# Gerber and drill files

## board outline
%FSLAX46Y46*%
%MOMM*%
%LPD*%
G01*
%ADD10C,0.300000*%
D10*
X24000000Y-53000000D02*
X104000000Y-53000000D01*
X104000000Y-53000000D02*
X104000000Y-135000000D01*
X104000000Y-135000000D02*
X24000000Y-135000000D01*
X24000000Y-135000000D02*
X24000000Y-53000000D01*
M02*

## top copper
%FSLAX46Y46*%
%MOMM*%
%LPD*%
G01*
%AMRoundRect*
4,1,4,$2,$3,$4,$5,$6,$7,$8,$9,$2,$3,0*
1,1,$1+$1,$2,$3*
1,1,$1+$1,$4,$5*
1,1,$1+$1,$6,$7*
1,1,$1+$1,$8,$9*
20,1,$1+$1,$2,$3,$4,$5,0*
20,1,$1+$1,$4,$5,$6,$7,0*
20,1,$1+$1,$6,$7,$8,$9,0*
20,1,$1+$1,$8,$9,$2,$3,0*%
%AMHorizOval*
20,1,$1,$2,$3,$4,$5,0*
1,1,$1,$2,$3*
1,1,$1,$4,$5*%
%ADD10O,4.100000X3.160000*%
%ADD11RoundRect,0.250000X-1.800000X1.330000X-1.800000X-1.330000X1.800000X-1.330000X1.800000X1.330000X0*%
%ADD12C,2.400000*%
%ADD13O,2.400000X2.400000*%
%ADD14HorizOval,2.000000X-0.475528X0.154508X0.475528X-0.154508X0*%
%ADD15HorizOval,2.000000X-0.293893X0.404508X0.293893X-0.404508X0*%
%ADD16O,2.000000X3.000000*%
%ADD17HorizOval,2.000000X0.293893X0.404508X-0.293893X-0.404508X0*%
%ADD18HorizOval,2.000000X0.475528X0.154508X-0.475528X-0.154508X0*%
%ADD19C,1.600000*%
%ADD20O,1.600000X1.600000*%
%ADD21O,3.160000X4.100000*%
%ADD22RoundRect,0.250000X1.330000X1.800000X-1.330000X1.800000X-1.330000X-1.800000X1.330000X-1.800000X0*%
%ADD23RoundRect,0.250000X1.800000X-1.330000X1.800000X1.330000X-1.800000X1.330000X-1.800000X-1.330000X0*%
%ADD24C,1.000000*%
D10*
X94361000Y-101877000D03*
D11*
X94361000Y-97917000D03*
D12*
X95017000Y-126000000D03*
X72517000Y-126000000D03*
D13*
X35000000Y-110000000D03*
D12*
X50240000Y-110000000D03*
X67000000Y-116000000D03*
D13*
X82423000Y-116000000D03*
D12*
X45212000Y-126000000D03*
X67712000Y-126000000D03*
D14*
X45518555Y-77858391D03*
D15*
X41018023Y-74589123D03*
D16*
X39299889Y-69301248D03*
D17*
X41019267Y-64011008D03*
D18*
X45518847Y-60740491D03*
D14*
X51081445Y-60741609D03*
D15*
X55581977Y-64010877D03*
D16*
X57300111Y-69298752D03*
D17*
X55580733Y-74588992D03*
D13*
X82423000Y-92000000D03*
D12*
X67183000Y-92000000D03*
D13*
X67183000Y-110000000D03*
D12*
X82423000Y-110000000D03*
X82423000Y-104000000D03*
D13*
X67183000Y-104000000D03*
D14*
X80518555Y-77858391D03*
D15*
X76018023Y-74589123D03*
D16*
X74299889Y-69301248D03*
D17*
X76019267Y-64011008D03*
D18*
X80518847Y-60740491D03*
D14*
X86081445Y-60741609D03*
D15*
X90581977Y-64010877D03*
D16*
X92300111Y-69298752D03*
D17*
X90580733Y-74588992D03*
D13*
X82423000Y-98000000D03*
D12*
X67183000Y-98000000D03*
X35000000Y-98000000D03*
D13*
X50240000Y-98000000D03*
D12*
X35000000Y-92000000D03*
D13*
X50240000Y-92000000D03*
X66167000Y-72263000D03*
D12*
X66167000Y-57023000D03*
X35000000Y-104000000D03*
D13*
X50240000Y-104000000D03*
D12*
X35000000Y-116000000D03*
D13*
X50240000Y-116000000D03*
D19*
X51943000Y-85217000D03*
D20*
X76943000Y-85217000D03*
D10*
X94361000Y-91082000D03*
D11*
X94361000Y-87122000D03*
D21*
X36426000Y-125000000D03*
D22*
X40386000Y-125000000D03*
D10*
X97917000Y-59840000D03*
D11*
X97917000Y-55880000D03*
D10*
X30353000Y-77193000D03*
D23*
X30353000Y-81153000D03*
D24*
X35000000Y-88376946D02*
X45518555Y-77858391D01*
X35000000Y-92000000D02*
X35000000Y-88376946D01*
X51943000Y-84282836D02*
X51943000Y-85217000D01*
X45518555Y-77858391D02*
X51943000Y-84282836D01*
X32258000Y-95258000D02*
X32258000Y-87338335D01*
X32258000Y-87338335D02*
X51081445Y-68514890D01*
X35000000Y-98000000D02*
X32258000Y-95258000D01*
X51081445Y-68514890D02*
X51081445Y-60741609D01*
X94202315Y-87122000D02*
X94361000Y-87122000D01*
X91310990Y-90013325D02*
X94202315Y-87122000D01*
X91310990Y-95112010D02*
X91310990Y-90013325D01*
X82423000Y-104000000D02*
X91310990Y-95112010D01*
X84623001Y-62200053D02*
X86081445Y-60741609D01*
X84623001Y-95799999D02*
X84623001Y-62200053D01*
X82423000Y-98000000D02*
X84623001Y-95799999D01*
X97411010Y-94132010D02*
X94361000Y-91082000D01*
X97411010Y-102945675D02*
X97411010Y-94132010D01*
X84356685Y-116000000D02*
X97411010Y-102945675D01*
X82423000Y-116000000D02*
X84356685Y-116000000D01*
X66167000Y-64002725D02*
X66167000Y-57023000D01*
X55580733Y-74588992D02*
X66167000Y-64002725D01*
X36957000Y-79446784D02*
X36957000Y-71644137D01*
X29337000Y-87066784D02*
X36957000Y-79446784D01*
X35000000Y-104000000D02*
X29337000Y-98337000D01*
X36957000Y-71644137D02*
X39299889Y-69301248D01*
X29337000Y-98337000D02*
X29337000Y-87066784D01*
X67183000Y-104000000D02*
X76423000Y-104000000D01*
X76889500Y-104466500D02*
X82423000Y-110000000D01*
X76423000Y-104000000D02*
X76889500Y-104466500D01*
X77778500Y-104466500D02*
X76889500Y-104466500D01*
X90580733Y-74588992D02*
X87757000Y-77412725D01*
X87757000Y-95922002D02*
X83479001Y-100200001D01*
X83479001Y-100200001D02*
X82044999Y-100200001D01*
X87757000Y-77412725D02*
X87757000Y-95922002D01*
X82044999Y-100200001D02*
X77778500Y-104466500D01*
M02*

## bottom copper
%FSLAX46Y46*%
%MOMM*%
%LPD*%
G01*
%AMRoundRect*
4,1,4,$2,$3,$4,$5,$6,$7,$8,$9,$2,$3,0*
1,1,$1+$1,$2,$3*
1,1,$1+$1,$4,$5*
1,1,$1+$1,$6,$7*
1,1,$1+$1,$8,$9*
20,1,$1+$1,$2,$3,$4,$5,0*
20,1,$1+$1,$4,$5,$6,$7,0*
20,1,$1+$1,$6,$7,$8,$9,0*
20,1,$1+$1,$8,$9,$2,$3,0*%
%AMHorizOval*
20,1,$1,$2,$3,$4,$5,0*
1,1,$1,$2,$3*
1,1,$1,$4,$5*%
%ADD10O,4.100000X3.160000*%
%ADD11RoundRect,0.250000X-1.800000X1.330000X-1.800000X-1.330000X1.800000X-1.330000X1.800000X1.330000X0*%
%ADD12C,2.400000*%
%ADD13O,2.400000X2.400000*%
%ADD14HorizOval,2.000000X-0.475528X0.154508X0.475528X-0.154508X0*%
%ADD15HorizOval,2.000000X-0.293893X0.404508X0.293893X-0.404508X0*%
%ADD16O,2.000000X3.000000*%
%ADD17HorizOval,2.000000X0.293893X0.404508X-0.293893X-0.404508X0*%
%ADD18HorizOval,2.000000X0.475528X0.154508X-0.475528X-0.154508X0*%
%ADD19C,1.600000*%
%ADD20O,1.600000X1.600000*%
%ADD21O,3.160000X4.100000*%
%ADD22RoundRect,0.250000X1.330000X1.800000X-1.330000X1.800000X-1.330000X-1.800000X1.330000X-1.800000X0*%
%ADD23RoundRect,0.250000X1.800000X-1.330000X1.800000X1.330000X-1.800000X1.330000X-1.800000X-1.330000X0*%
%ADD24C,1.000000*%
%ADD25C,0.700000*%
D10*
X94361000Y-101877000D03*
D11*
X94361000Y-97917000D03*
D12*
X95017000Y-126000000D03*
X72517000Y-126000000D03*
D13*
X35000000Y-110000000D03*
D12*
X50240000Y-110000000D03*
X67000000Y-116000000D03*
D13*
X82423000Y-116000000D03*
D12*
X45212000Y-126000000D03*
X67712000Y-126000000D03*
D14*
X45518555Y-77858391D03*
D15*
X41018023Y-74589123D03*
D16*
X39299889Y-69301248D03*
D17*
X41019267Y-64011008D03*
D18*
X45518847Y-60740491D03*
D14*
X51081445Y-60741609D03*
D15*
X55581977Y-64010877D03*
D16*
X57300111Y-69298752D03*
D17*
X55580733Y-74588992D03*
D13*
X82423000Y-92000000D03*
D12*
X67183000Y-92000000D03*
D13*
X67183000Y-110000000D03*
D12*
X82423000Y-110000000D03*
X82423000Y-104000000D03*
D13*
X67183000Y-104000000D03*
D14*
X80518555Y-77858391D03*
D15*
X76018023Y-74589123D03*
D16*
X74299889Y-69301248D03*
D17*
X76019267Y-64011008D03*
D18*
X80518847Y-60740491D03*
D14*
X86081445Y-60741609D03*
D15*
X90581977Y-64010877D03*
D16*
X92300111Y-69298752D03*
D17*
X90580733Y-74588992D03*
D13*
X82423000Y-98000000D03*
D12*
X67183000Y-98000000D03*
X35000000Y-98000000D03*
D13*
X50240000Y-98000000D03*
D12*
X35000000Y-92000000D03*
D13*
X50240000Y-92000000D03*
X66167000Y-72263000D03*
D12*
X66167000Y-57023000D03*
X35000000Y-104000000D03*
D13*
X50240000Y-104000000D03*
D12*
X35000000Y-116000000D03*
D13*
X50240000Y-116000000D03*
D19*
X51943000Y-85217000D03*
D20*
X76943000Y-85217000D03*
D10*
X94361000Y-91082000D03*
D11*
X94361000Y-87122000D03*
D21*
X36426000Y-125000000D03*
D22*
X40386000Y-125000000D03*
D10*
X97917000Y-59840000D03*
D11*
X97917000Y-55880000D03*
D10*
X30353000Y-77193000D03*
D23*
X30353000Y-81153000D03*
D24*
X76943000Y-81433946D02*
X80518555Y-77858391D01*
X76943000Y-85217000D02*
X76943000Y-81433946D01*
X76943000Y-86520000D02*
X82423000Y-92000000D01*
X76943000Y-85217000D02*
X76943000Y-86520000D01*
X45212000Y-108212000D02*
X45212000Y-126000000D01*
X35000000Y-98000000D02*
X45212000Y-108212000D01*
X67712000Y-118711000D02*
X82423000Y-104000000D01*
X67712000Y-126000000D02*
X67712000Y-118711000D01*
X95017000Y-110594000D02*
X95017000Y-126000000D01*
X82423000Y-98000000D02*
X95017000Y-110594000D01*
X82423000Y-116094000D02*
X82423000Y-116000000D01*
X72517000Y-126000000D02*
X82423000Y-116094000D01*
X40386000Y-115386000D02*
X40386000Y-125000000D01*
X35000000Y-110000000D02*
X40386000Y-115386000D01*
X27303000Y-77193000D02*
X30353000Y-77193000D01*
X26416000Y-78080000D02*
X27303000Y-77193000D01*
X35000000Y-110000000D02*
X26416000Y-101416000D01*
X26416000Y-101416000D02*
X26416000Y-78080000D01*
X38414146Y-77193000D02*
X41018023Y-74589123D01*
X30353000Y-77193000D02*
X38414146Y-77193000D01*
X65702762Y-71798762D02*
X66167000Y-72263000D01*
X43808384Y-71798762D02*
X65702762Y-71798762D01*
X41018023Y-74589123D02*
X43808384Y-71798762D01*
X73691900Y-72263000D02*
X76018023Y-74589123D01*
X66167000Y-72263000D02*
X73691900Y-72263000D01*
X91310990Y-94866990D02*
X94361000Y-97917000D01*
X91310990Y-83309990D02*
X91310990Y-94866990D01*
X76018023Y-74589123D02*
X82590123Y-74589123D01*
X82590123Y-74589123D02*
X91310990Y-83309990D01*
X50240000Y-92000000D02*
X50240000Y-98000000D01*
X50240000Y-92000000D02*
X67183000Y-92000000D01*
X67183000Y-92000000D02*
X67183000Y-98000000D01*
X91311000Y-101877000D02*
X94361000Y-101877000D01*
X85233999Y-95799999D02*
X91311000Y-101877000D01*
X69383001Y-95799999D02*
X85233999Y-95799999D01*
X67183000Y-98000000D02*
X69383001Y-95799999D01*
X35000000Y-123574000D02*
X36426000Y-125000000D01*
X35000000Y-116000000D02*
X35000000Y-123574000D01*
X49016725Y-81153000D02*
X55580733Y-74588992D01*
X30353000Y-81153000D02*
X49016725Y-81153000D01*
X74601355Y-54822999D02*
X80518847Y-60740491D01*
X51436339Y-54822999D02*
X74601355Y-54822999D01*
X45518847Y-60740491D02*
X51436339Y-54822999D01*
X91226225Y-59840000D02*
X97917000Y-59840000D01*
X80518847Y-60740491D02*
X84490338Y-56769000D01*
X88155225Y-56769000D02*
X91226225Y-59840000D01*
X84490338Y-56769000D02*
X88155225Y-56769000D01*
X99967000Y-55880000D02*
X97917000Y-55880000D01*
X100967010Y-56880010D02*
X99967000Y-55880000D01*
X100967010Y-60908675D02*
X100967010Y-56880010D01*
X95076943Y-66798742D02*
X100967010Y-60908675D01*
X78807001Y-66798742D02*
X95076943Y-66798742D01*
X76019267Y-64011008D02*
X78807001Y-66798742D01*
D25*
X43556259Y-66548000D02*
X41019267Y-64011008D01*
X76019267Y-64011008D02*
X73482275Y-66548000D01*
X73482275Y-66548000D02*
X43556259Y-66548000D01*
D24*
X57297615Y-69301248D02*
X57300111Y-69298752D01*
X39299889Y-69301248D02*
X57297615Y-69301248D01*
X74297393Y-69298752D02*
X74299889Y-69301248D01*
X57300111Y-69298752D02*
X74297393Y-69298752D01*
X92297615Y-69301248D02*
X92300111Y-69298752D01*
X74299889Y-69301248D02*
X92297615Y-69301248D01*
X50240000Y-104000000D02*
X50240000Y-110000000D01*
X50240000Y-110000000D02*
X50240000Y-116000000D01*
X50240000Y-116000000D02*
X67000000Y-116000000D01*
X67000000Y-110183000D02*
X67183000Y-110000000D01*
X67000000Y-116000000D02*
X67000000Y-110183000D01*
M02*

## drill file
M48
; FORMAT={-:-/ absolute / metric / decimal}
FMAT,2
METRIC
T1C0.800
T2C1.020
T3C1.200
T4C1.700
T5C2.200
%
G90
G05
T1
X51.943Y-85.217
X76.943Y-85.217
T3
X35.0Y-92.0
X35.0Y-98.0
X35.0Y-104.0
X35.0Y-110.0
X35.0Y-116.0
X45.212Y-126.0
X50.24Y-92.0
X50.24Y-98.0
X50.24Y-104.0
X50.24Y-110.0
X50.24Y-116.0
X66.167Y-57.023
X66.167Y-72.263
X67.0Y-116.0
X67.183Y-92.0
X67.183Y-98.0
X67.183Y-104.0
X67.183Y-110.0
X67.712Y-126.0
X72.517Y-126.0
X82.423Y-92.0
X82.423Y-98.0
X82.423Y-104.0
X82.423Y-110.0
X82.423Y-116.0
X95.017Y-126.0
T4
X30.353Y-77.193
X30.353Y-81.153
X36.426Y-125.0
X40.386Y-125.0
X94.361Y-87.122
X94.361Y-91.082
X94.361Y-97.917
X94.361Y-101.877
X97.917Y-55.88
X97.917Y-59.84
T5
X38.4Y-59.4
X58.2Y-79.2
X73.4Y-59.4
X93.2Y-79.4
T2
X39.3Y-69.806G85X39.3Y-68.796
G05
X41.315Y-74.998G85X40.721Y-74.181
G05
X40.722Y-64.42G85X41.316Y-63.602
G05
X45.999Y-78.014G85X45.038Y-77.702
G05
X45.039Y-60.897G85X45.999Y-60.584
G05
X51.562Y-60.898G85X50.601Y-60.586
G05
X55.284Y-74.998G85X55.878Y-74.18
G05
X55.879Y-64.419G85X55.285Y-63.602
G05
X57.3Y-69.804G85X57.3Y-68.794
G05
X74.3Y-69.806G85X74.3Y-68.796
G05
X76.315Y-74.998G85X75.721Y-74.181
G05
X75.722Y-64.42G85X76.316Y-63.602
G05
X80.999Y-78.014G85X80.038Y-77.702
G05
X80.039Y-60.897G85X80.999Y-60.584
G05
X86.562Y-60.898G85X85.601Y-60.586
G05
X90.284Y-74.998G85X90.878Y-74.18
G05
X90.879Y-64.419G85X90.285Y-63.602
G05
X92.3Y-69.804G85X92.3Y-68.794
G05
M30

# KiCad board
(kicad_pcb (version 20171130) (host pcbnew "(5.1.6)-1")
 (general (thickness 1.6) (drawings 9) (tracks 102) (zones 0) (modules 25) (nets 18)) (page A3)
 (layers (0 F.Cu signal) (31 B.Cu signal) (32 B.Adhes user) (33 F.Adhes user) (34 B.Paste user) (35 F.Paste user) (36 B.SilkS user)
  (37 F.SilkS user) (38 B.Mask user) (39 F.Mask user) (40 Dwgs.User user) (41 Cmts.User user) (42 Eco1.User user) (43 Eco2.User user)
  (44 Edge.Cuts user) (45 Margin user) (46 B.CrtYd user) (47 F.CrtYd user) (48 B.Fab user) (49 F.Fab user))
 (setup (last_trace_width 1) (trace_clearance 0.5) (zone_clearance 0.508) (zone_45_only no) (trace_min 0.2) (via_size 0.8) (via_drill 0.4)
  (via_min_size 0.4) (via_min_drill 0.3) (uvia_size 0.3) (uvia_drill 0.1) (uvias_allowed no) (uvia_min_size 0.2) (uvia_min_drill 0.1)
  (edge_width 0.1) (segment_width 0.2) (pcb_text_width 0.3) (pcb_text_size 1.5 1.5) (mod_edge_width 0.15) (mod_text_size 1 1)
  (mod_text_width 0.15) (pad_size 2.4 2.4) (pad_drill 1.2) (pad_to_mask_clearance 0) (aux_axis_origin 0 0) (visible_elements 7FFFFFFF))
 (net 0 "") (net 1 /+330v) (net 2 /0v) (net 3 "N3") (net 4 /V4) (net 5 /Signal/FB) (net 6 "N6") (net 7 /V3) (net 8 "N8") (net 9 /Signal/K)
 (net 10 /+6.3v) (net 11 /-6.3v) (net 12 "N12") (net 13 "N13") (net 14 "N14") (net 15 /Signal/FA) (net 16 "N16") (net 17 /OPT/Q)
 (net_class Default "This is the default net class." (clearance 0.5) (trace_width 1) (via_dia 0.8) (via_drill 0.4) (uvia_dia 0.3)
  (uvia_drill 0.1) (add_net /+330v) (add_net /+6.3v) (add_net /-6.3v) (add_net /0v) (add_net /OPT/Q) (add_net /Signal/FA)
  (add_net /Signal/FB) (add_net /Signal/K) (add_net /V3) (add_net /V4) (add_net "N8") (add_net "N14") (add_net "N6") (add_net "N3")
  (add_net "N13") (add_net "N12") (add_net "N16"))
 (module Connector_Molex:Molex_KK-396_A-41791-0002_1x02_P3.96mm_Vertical (layer F.Cu) (at 94.361 97.917 270)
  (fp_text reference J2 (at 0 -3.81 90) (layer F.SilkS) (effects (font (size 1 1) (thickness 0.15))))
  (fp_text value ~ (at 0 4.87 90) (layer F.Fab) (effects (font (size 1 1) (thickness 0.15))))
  (pad 2 thru_hole oval (at 3.96 0 270) (size 3.16 4.1) (drill 1.7) (layers *.Cu *.Mask) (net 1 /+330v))
  (pad 1 thru_hole roundrect (at 0 0 270) (size 3.16 4.1) (drill 1.7) (layers *.Cu *.Mask) (roundrect_rratio 0.079114) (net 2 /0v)))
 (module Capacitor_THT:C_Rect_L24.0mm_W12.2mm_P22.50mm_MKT (layer F.Cu) (at 72.517 126)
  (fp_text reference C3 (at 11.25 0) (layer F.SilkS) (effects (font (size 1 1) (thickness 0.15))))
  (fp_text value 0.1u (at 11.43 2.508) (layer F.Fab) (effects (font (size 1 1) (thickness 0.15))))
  (pad 2 thru_hole circle (at 22.5 0) (size 2.4 2.4) (drill 1.2) (layers *.Cu *.Mask) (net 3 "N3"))
  (pad 1 thru_hole circle (at 0 0) (size 2.4 2.4) (drill 1.2) (layers *.Cu *.Mask) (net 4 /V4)))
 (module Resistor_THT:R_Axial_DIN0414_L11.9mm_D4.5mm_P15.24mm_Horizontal (layer F.Cu) (at 50.24 110 180)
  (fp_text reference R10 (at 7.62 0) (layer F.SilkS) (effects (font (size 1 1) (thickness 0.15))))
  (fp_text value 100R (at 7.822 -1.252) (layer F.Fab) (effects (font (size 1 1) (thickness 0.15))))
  (pad 2 thru_hole oval (at 15.24 0 180) (size 2.4 2.4) (drill 1.2) (layers *.Cu *.Mask) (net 2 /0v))
  (pad 1 thru_hole circle (at 0 0 180) (size 2.4 2.4) (drill 1.2) (layers *.Cu *.Mask) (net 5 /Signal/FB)))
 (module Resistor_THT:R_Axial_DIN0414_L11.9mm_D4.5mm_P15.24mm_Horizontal (layer F.Cu) (at 67.183 116)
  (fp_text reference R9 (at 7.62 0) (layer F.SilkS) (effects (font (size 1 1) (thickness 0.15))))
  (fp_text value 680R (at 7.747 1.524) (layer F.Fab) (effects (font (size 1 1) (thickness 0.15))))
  (pad 1 thru_hole circle (at -0.183 0) (size 2.4 2.4) (drill 1.2) (layers *.Cu *.Mask) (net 5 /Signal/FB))
  (pad 2 thru_hole oval (at 15.24 0) (size 2.4 2.4) (drill 1.2) (layers *.Cu *.Mask) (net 4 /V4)))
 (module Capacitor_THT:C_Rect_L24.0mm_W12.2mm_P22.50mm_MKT (layer F.Cu) (at 45.212 126)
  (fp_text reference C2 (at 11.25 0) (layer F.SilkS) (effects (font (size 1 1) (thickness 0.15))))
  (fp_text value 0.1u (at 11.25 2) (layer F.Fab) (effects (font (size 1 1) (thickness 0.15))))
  (pad 1 thru_hole circle (at 0 0) (size 2.4 2.4) (drill 1.2) (layers *.Cu *.Mask) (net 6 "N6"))
  (pad 2 thru_hole circle (at 22.5 0) (size 2.4 2.4) (drill 1.2) (layers *.Cu *.Mask) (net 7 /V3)))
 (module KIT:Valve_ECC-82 (layer B.Cu) (at 48.3 69.3 198)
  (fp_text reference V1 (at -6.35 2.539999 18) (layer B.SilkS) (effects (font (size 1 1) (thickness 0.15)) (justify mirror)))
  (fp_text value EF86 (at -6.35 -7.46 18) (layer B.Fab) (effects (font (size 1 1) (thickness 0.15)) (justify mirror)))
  (pad 1 thru_hole oval (at 5.29 -7.28 252) (size 2 3) (drill oval 1.02 2.03) (layers *.Cu *.Mask) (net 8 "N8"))
  (pad 2 thru_hole oval (at 8.56 -2.78 216) (size 2 3) (drill oval 1.02 2.03) (layers *.Cu *.Mask) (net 2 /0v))
  (pad 3 thru_hole oval (at 8.56 2.78 180) (size 2 3) (drill oval 1.02 2.03) (layers *.Cu *.Mask) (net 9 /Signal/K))
  (pad 4 thru_hole oval (at 5.29 7.28 144) (size 2 3) (drill oval 1.02 2.03) (layers *.Cu *.Mask) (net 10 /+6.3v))
  (pad 5 thru_hole oval (at 0 9 108) (size 2 3) (drill oval 1.02 2.03) (layers *.Cu *.Mask) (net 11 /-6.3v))
  (pad 6 thru_hole oval (at -5.29 7.28 252) (size 2 3) (drill oval 1.02 2.03) (layers *.Cu *.Mask) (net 6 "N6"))
  (pad 7 thru_hole oval (at -8.56 2.78 216) (size 2 3) (drill oval 1.02 2.03) (layers *.Cu *.Mask) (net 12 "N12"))
  (pad 8 thru_hole oval (at -8.56 -2.78 180) (size 2 3) (drill oval 1.02 2.03) (layers *.Cu *.Mask) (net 9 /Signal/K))
  (pad 9 thru_hole oval (at -5.29 -7.28 144) (size 2 3) (drill oval 1.02 2.03) (layers *.Cu *.Mask) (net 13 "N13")))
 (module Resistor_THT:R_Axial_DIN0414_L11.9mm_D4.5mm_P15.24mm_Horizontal (layer F.Cu) (at 67.183 92)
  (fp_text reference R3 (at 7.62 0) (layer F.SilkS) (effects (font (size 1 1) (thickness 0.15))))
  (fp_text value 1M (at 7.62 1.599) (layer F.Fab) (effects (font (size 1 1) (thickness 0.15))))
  (pad 2 thru_hole oval (at 15.24 0) (size 2.4 2.4) (drill 1.2) (layers *.Cu *.Mask) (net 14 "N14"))
  (pad 1 thru_hole circle (at 0 0) (size 2.4 2.4) (drill 1.2) (layers *.Cu *.Mask) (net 1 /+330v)))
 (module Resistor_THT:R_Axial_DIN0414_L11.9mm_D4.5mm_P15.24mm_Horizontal (layer F.Cu) (at 82.423 110 180)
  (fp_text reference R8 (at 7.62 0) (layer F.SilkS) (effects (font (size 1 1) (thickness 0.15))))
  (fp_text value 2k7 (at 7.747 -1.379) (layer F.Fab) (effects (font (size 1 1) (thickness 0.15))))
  (pad 2 thru_hole oval (at 15.24 0 180) (size 2.4 2.4) (drill 1.2) (layers *.Cu *.Mask) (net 5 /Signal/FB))
  (pad 1 thru_hole circle (at 0 0 180) (size 2.4 2.4) (drill 1.2) (layers *.Cu *.Mask) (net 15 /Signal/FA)))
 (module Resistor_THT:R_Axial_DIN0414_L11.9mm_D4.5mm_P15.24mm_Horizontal (layer F.Cu) (at 82.423 104 180)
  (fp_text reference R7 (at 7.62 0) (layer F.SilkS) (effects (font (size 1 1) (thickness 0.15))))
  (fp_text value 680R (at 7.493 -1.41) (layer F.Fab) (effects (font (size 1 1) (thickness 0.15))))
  (pad 1 thru_hole circle (at 0 0 180) (size 2.4 2.4) (drill 1.2) (layers *.Cu *.Mask) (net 7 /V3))
  (pad 2 thru_hole oval (at 15.24 0 180) (size 2.4 2.4) (drill 1.2) (layers *.Cu *.Mask) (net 15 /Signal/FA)))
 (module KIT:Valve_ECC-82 (layer B.Cu) (at 83.3 69.3 198)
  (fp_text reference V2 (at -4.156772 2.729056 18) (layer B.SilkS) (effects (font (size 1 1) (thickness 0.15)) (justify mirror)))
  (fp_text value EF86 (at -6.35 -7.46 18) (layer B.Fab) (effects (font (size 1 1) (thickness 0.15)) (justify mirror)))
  (pad 1 thru_hole oval (at 5.29 -7.28 252) (size 2 3) (drill oval 1.02 2.03) (layers *.Cu *.Mask) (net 14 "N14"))
  (pad 2 thru_hole oval (at 8.56 -2.78 216) (size 2 3) (drill oval 1.02 2.03) (layers *.Cu *.Mask) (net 2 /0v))
  (pad 3 thru_hole oval (at 8.56 2.78 180) (size 2 3) (drill oval 1.02 2.03) (layers *.Cu *.Mask) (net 9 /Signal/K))
  (pad 4 thru_hole oval (at 5.29 7.28 144) (size 2 3) (drill oval 1.02 2.03) (layers *.Cu *.Mask) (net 10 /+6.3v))
  (pad 5 thru_hole oval (at 0 9 108) (size 2 3) (drill oval 1.02 2.03) (layers *.Cu *.Mask) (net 11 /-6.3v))
  (pad 6 thru_hole oval (at -5.29 7.28 252) (size 2 3) (drill oval 1.02 2.03) (layers *.Cu *.Mask) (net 3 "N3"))
  (pad 7 thru_hole oval (at -8.56 2.78 216) (size 2 3) (drill oval 1.02 2.03) (layers *.Cu *.Mask) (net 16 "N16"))
  (pad 8 thru_hole oval (at -8.56 -2.78 180) (size 2 3) (drill oval 1.02 2.03) (layers *.Cu *.Mask) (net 9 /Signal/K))
  (pad 9 thru_hole oval (at -5.29 -7.28 144) (size 2 3) (drill oval 1.02 2.03) (layers *.Cu *.Mask) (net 15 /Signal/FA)))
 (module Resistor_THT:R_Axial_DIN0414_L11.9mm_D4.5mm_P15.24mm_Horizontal (layer F.Cu) (at 67.183 98)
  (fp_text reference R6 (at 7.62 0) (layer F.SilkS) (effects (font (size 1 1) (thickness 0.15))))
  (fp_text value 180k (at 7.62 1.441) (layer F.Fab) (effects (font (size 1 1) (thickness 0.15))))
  (pad 2 thru_hole oval (at 15.24 0) (size 2.4 2.4) (drill 1.2) (layers *.Cu *.Mask) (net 3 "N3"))
  (pad 1 thru_hole circle (at 0 0) (size 2.4 2.4) (drill 1.2) (layers *.Cu *.Mask) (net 1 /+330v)))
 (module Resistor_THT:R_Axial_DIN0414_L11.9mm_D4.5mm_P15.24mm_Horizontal (layer F.Cu) (at 35 98)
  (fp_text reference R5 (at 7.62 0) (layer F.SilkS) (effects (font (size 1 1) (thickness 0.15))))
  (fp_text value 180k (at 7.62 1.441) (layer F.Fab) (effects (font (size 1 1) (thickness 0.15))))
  (pad 1 thru_hole circle (at 0 0) (size 2.4 2.4) (drill 1.2) (layers *.Cu *.Mask) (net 6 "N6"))
  (pad 2 thru_hole oval (at 15.24 0) (size 2.4 2.4) (drill 1.2) (layers *.Cu *.Mask) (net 1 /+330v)))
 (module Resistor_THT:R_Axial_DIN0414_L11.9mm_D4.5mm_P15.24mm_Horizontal (layer F.Cu) (at 35 92)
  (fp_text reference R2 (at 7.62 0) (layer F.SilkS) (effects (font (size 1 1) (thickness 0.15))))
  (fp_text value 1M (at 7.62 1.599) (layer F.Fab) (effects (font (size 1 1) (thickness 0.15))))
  (pad 1 thru_hole circle (at 0 0) (size 2.4 2.4) (drill 1.2) (layers *.Cu *.Mask) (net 8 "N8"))
  (pad 2 thru_hole oval (at 15.24 0) (size 2.4 2.4) (drill 1.2) (layers *.Cu *.Mask) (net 1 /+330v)))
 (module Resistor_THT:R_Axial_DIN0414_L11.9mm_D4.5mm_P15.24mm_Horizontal (layer F.Cu) (at 66.167 57.023 270)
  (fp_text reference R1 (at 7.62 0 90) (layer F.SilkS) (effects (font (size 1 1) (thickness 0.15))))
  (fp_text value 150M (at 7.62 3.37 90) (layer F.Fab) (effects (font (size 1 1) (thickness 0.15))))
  (pad 2 thru_hole oval (at 15.24 0 270) (size 2.4 2.4) (drill 1.2) (layers *.Cu *.Mask) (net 2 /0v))
  (pad 1 thru_hole circle (at 0 0 270) (size 2.4 2.4) (drill 1.2) (layers *.Cu *.Mask) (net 13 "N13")))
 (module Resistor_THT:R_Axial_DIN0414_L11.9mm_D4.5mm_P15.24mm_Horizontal (layer F.Cu) (at 35 104)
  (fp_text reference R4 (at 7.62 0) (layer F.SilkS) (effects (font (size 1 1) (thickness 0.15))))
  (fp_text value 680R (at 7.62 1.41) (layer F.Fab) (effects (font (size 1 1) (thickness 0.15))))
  (pad 1 thru_hole circle (at 0 0) (size 2.4 2.4) (drill 1.2) (layers *.Cu *.Mask) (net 9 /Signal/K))
  (pad 2 thru_hole oval (at 15.24 0) (size 2.4 2.4) (drill 1.2) (layers *.Cu *.Mask) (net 5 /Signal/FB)))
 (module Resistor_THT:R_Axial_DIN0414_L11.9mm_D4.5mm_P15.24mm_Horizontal (layer F.Cu) (at 35 116)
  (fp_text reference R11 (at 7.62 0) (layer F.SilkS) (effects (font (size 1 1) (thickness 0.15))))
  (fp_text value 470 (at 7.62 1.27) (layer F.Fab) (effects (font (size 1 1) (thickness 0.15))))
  (pad 1 thru_hole circle (at 0 0) (size 2.4 2.4) (drill 1.2) (layers *.Cu *.Mask) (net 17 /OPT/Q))
  (pad 2 thru_hole oval (at 15.24 0) (size 2.4 2.4) (drill 1.2) (layers *.Cu *.Mask) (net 5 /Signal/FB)))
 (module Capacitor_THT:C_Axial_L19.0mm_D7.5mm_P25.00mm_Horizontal (layer F.Cu) (at 51.943 85.217)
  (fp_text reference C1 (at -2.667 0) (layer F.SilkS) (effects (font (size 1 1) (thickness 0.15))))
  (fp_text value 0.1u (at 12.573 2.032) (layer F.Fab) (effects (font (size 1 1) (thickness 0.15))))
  (pad 1 thru_hole circle (at 0 0) (size 1.6 1.6) (drill 0.8) (layers *.Cu *.Mask) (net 8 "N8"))
  (pad 2 thru_hole oval (at 25 0) (size 1.6 1.6) (drill 0.8) (layers *.Cu *.Mask) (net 14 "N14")))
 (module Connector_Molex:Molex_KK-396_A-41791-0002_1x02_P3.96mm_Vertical (layer F.Cu) (at 94.361 87.122 270)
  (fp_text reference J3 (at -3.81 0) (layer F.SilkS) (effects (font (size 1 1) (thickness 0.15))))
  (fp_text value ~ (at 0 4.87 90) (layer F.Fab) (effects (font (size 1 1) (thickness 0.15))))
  (pad 2 thru_hole oval (at 3.96 0 270) (size 3.16 4.1) (drill 1.7) (layers *.Cu *.Mask) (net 4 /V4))
  (pad 1 thru_hole roundrect (at 0 0 270) (size 3.16 4.1) (drill 1.7) (layers *.Cu *.Mask) (roundrect_rratio 0.079114) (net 7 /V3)))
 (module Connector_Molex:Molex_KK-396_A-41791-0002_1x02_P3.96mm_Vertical (layer F.Cu) (at 40.386 125 180)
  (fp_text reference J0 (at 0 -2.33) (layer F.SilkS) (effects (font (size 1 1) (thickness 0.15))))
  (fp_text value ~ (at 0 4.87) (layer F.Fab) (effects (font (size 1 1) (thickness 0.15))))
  (pad 2 thru_hole oval (at 3.96 0 180) (size 3.16 4.1) (drill 1.7) (layers *.Cu *.Mask) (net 17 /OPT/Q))
  (pad 1 thru_hole roundrect (at 0 0 180) (size 3.16 4.1) (drill 1.7) (layers *.Cu *.Mask) (roundrect_rratio 0.079114) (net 2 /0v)))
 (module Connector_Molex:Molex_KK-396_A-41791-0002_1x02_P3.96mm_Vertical (layer F.Cu) (at 97.917 55.88 270)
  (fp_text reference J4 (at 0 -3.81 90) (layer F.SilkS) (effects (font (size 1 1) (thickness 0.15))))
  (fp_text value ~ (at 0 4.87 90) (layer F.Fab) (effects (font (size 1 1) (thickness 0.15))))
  (pad 2 thru_hole oval (at 3.96 0 270) (size 3.16 4.1) (drill 1.7) (layers *.Cu *.Mask) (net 11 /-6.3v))
  (pad 1 thru_hole roundrect (at 0 0 270) (size 3.16 4.1) (drill 1.7) (layers *.Cu *.Mask) (roundrect_rratio 0.079114) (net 10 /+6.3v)))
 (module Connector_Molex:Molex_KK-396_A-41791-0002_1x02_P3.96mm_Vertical (layer F.Cu) (at 30.353 81.153 90)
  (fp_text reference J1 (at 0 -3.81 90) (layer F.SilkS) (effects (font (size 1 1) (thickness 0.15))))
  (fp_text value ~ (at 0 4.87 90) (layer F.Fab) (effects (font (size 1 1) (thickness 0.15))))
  (pad 2 thru_hole oval (at 3.96 0 90) (size 3.16 4.1) (drill 1.7) (layers *.Cu *.Mask) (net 2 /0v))
  (pad 1 thru_hole roundrect (at 0 0 90) (size 3.16 4.1) (drill 1.7) (layers *.Cu *.Mask) (roundrect_rratio 0.079114) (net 13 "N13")))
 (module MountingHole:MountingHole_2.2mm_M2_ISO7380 (layer F.Cu) (at 38.4 59.4)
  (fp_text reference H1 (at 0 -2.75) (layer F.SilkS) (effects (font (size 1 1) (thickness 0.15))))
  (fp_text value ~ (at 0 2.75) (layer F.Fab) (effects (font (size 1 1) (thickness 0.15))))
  (pad 1 np_thru_hole circle (at 0 0) (size 2.2 2.2) (drill 2.2) (layers *.Cu *.Mask)))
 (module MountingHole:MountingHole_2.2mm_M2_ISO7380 (layer F.Cu) (at 58.2 79.2)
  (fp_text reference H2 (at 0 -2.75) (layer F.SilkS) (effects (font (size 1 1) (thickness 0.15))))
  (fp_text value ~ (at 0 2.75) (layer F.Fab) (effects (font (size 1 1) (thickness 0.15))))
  (pad 1 np_thru_hole circle (at 0 0) (size 2.2 2.2) (drill 2.2) (layers *.Cu *.Mask)))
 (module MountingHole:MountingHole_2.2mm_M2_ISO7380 (layer F.Cu) (at 73.4 59.4)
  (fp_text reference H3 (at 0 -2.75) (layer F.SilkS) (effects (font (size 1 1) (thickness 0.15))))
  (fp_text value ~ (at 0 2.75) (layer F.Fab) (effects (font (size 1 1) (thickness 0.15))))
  (pad 1 np_thru_hole circle (at 0 0) (size 2.2 2.2) (drill 2.2) (layers *.Cu *.Mask)))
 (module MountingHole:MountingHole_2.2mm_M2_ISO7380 (layer F.Cu) (at 93.2 79.4)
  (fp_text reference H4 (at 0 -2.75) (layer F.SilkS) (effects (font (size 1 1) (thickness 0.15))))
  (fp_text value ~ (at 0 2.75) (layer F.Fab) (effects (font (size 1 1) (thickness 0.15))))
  (pad 1 np_thru_hole circle (at 0 0) (size 2.2 2.2) (drill 2.2) (layers *.Cu *.Mask)))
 (gr_line (start 24 53) (end 104 53) (layer Edge.Cuts) (width 0.3))
 (gr_line (start 104 53) (end 104 135) (layer Edge.Cuts) (width 0.3))
 (gr_line (start 104 135) (end 24 135) (layer Edge.Cuts) (width 0.3))
 (gr_line (start 24 135) (end 24 53) (layer Edge.Cuts) (width 0.3))
 (segment (start 35 88.376946) (end 45.518555 77.858391) (width 1) (layer F.Cu) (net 8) (status 20))
 (segment (start 35 92) (end 35 88.376946) (width 1) (layer F.Cu) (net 8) (status 10))
 (segment (start 51.943 84.282836) (end 51.943 85.217) (width 1) (layer F.Cu) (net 8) (status 20))
 (segment (start 45.518555 77.858391) (end 51.943 84.282836) (width 1) (layer F.Cu) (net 8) (status 10))
 (segment (start 76.943 81.433946) (end 80.518555 77.858391) (width 1) (layer B.Cu) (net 14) (status 20))
 (segment (start 76.943 85.217) (end 76.943 81.433946) (width 1) (layer B.Cu) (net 14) (status 10))
 (segment (start 76.943 86.52) (end 82.423 92) (width 1) (layer B.Cu) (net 14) (status 20))
 (segment (start 76.943 85.217) (end 76.943 86.52) (width 1) (layer B.Cu) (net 14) (status 10))
 (segment (start 32.258 95.258) (end 32.258 87.338335) (width 1) (layer F.Cu) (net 6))
 (segment (start 32.258 87.338335) (end 51.081445 68.51489) (width 1) (layer F.Cu) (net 6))
 (segment (start 35 98) (end 32.258 95.258) (width 1) (layer F.Cu) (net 6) (status 10))
 (segment (start 51.081445 68.51489) (end 51.081445 60.741609) (width 1) (layer F.Cu) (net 6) (status 20))
 (segment (start 45.212 108.212) (end 45.212 126) (width 1) (layer B.Cu) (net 6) (status 20))
 (segment (start 35 98) (end 45.212 108.212) (width 1) (layer B.Cu) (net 6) (status 10))
 (segment (start 67.712 118.711) (end 82.423 104) (width 1) (layer B.Cu) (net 7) (status 20))
 (segment (start 67.712 126) (end 67.712 118.711) (width 1) (layer B.Cu) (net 7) (status 10))
 (segment (start 94.202315 87.122) (end 94.361 87.122) (width 1) (layer F.Cu) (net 7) (status 30))
 (segment (start 91.31099 90.013325) (end 94.202315 87.122) (width 1) (layer F.Cu) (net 7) (status 20))
 (segment (start 91.31099 95.11201) (end 91.31099 90.013325) (width 1) (layer F.Cu) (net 7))
 (segment (start 82.423 104) (end 91.31099 95.11201) (width 1) (layer F.Cu) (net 7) (status 10))
 (segment (start 95.017 110.594) (end 95.017 126) (width 1) (layer B.Cu) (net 3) (status 20))
 (segment (start 82.423 98) (end 95.017 110.594) (width 1) (layer B.Cu) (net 3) (status 10))
 (segment (start 84.623001 62.200053) (end 86.081445 60.741609) (width 1) (layer F.Cu) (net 3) (status 20))
 (segment (start 84.623001 95.799999) (end 84.623001 62.200053) (width 1) (layer F.Cu) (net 3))
 (segment (start 82.423 98) (end 84.623001 95.799999) (width 1) (layer F.Cu) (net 3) (status 10))
 (segment (start 82.423 116.094) (end 82.423 116) (width 1) (layer B.Cu) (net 4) (status 30))
 (segment (start 72.517 126) (end 82.423 116.094) (width 1) (layer B.Cu) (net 4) (status 30))
 (segment (start 97.41101 94.13201) (end 94.361 91.082) (width 1) (layer F.Cu) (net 4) (status 20))
 (segment (start 97.41101 102.945675) (end 97.41101 94.13201) (width 1) (layer F.Cu) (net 4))
 (segment (start 84.356685 116) (end 97.41101 102.945675) (width 1) (layer F.Cu) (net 4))
 (segment (start 82.423 116) (end 84.356685 116) (width 1) (layer F.Cu) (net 4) (status 10))
 (segment (start 40.386 115.386) (end 40.386 125) (width 1) (layer B.Cu) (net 2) (status 20))
 (segment (start 35 110) (end 40.386 115.386) (width 1) (layer B.Cu) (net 2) (status 10))
 (segment (start 27.303 77.193) (end 30.353 77.193) (width 1) (layer B.Cu) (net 2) (status 20))
 (segment (start 26.416 78.08) (end 27.303 77.193) (width 1) (layer B.Cu) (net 2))
 (segment (start 35 110) (end 26.416 101.416) (width 1) (layer B.Cu) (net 2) (status 10))
 (segment (start 26.416 101.416) (end 26.416 78.08) (width 1) (layer B.Cu) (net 2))
 (segment (start 38.414146 77.193) (end 41.018023 74.589123) (width 1) (layer B.Cu) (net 2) (status 20))
 (segment (start 30.353 77.193) (end 38.414146 77.193) (width 1) (layer B.Cu) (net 2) (status 10))
 (segment (start 65.702762 71.798762) (end 66.167 72.263) (width 1) (layer B.Cu) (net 2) (status 30))
 (segment (start 43.808384 71.798762) (end 65.702762 71.798762) (width 1) (layer B.Cu) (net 2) (status 20))
 (segment (start 41.018023 74.589123) (end 43.808384 71.798762) (width 1) (layer B.Cu) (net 2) (status 10))
 (segment (start 73.6919 72.263) (end 76.018023 74.589123) (width 1) (layer B.Cu) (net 2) (status 20))
 (segment (start 66.167 72.263) (end 73.6919 72.263) (width 1) (layer B.Cu) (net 2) (status 10))
 (segment (start 91.31099 94.86699) (end 94.361 97.917) (width 1) (layer B.Cu) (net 2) (status 20))
 (segment (start 91.31099 83.30999) (end 91.31099 94.86699) (width 1) (layer B.Cu) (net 2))
 (segment (start 76.018023 74.589123) (end 82.590123 74.589123) (width 1) (layer B.Cu) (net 2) (status 10))
 (segment (start 82.590123 74.589123) (end 91.31099 83.30999) (width 1) (layer B.Cu) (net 2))
 (segment (start 50.24 92) (end 50.24 98) (width 1) (layer B.Cu) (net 1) (status 30))
 (segment (start 50.24 92) (end 67.183 92) (width 1) (layer B.Cu) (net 1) (status 30))
 (segment (start 67.183 92) (end 67.183 98) (width 1) (layer B.Cu) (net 1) (status 30))
 (segment (start 91.311 101.877) (end 94.361 101.877) (width 1) (layer B.Cu) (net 1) (status 20))
 (segment (start 85.233999 95.799999) (end 91.311 101.877) (width 1) (layer B.Cu) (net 1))
 (segment (start 69.383001 95.799999) (end 85.233999 95.799999) (width 1) (layer B.Cu) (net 1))
 (segment (start 67.183 98) (end 69.383001 95.799999) (width 1) (layer B.Cu) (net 1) (status 10))
 (segment (start 35 123.574) (end 36.426 125) (width 1) (layer B.Cu) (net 17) (status 20))
 (segment (start 35 116) (end 35 123.574) (width 1) (layer B.Cu) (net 17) (status 10))
 (segment (start 49.016725 81.153) (end 55.580733 74.588992) (width 1) (layer B.Cu) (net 13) (status 20))
 (segment (start 30.353 81.153) (end 49.016725 81.153) (width 1) (layer B.Cu) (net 13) (status 10))
 (segment (start 66.167 64.002725) (end 66.167 57.023) (width 1) (layer F.Cu) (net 13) (status 20))
 (segment (start 55.580733 74.588992) (end 66.167 64.002725) (width 1) (layer F.Cu) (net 13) (status 10))
 (segment (start 74.601355 54.822999) (end 80.518847 60.740491) (width 1) (layer B.Cu) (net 11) (status 20))
 (segment (start 51.436339 54.822999) (end 74.601355 54.822999) (width 1) (layer B.Cu) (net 11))
 (segment (start 45.518847 60.740491) (end 51.436339 54.822999) (width 1) (layer B.Cu) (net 11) (status 10))
 (segment (start 91.226225 59.84) (end 97.917 59.84) (width 1) (layer B.Cu) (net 11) (status 20))
 (segment (start 80.518847 60.740491) (end 84.490338 56.769) (width 1) (layer B.Cu) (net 11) (status 10))
 (segment (start 88.155225 56.769) (end 91.226225 59.84) (width 1) (layer B.Cu) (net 11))
 (segment (start 84.490338 56.769) (end 88.155225 56.769) (width 1) (layer B.Cu) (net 11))
 (segment (start 99.967 55.88) (end 97.917 55.88) (width 1) (layer B.Cu) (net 10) (status 20))
 (segment (start 100.96701 56.88001) (end 99.967 55.88) (width 1) (layer B.Cu) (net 10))
 (segment (start 100.96701 60.908675) (end 100.96701 56.88001) (width 1) (layer B.Cu) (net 10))
 (segment (start 95.076943 66.798742) (end 100.96701 60.908675) (width 1) (layer B.Cu) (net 10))
 (segment (start 78.807001 66.798742) (end 95.076943 66.798742) (width 1) (layer B.Cu) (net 10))
 (segment (start 76.019267 64.011008) (end 78.807001 66.798742) (width 1) (layer B.Cu) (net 10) (status 10))
 (segment (start 43.556259 66.548) (end 41.019267 64.011008) (width 0.7) (layer B.Cu) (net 10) (status 20))
 (segment (start 76.019267 64.011008) (end 73.482275 66.548) (width 0.7) (layer B.Cu) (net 10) (status 10))
 (segment (start 73.482275 66.548) (end 43.556259 66.548) (width 0.7) (layer B.Cu) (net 10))
 (segment (start 57.297615 69.301248) (end 57.300111 69.298752) (width 1) (layer B.Cu) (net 9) (status 30))
 (segment (start 39.299889 69.301248) (end 57.297615 69.301248) (width 1) (layer B.Cu) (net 9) (status 30))
 (segment (start 74.297393 69.298752) (end 74.299889 69.301248) (width 1) (layer B.Cu) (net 9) (status 30))
 (segment (start 57.300111 69.298752) (end 74.297393 69.298752) (width 1) (layer B.Cu) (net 9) (status 30))
 (segment (start 92.297615 69.301248) (end 92.300111 69.298752) (width 1) (layer B.Cu) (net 9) (status 30))
 (segment (start 74.299889 69.301248) (end 92.297615 69.301248) (width 1) (layer B.Cu) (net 9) (status 30))
 (segment (start 36.957 79.446784) (end 36.957 71.644137) (width 1) (layer F.Cu) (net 9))
 (segment (start 29.337 87.066784) (end 36.957 79.446784) (width 1) (layer F.Cu) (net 9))
 (segment (start 35 104) (end 29.337 98.337) (width 1) (layer F.Cu) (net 9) (status 10))
 (segment (start 36.957 71.644137) (end 39.299889 69.301248) (width 1) (layer F.Cu) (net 9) (status 20))
 (segment (start 29.337 98.337) (end 29.337 87.066784) (width 1) (layer F.Cu) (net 9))
 (segment (start 50.24 104) (end 50.24 110) (width 1) (layer B.Cu) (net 5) (status 30))
 (segment (start 50.24 110) (end 50.24 116) (width 1) (layer B.Cu) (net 5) (status 30))
 (segment (start 50.24 116) (end 67 116) (width 1) (layer B.Cu) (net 5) (status 30))
 (segment (start 67 110.183) (end 67.183 110) (width 1) (layer B.Cu) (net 5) (status 30))
 (segment (start 67 116) (end 67 110.183) (width 1) (layer B.Cu) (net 5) (status 30))
 (segment (start 67.183 104) (end 76.423 104) (width 1) (layer F.Cu) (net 15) (status 10))
 (segment (start 76.8895 104.4665) (end 82.423 110) (width 1) (layer F.Cu) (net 15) (status 20))
 (segment (start 76.423 104) (end 76.8895 104.4665) (width 1) (layer F.Cu) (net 15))
 (segment (start 77.7785 104.4665) (end 76.8895 104.4665) (width 1) (layer F.Cu) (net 15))
 (segment (start 90.580733 74.588992) (end 87.757 77.412725) (width 1) (layer F.Cu) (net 15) (status 10))
 (segment (start 87.757 95.922002) (end 83.479001 100.200001) (width 1) (layer F.Cu) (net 15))
 (segment (start 83.479001 100.200001) (end 82.044999 100.200001) (width 1) (layer F.Cu) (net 15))
 (segment (start 87.757 77.412725) (end 87.757 95.922002) (width 1) (layer F.Cu) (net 15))
 (segment (start 82.044999 100.200001) (end 77.7785 104.4665) (width 1) (layer F.Cu) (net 15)))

